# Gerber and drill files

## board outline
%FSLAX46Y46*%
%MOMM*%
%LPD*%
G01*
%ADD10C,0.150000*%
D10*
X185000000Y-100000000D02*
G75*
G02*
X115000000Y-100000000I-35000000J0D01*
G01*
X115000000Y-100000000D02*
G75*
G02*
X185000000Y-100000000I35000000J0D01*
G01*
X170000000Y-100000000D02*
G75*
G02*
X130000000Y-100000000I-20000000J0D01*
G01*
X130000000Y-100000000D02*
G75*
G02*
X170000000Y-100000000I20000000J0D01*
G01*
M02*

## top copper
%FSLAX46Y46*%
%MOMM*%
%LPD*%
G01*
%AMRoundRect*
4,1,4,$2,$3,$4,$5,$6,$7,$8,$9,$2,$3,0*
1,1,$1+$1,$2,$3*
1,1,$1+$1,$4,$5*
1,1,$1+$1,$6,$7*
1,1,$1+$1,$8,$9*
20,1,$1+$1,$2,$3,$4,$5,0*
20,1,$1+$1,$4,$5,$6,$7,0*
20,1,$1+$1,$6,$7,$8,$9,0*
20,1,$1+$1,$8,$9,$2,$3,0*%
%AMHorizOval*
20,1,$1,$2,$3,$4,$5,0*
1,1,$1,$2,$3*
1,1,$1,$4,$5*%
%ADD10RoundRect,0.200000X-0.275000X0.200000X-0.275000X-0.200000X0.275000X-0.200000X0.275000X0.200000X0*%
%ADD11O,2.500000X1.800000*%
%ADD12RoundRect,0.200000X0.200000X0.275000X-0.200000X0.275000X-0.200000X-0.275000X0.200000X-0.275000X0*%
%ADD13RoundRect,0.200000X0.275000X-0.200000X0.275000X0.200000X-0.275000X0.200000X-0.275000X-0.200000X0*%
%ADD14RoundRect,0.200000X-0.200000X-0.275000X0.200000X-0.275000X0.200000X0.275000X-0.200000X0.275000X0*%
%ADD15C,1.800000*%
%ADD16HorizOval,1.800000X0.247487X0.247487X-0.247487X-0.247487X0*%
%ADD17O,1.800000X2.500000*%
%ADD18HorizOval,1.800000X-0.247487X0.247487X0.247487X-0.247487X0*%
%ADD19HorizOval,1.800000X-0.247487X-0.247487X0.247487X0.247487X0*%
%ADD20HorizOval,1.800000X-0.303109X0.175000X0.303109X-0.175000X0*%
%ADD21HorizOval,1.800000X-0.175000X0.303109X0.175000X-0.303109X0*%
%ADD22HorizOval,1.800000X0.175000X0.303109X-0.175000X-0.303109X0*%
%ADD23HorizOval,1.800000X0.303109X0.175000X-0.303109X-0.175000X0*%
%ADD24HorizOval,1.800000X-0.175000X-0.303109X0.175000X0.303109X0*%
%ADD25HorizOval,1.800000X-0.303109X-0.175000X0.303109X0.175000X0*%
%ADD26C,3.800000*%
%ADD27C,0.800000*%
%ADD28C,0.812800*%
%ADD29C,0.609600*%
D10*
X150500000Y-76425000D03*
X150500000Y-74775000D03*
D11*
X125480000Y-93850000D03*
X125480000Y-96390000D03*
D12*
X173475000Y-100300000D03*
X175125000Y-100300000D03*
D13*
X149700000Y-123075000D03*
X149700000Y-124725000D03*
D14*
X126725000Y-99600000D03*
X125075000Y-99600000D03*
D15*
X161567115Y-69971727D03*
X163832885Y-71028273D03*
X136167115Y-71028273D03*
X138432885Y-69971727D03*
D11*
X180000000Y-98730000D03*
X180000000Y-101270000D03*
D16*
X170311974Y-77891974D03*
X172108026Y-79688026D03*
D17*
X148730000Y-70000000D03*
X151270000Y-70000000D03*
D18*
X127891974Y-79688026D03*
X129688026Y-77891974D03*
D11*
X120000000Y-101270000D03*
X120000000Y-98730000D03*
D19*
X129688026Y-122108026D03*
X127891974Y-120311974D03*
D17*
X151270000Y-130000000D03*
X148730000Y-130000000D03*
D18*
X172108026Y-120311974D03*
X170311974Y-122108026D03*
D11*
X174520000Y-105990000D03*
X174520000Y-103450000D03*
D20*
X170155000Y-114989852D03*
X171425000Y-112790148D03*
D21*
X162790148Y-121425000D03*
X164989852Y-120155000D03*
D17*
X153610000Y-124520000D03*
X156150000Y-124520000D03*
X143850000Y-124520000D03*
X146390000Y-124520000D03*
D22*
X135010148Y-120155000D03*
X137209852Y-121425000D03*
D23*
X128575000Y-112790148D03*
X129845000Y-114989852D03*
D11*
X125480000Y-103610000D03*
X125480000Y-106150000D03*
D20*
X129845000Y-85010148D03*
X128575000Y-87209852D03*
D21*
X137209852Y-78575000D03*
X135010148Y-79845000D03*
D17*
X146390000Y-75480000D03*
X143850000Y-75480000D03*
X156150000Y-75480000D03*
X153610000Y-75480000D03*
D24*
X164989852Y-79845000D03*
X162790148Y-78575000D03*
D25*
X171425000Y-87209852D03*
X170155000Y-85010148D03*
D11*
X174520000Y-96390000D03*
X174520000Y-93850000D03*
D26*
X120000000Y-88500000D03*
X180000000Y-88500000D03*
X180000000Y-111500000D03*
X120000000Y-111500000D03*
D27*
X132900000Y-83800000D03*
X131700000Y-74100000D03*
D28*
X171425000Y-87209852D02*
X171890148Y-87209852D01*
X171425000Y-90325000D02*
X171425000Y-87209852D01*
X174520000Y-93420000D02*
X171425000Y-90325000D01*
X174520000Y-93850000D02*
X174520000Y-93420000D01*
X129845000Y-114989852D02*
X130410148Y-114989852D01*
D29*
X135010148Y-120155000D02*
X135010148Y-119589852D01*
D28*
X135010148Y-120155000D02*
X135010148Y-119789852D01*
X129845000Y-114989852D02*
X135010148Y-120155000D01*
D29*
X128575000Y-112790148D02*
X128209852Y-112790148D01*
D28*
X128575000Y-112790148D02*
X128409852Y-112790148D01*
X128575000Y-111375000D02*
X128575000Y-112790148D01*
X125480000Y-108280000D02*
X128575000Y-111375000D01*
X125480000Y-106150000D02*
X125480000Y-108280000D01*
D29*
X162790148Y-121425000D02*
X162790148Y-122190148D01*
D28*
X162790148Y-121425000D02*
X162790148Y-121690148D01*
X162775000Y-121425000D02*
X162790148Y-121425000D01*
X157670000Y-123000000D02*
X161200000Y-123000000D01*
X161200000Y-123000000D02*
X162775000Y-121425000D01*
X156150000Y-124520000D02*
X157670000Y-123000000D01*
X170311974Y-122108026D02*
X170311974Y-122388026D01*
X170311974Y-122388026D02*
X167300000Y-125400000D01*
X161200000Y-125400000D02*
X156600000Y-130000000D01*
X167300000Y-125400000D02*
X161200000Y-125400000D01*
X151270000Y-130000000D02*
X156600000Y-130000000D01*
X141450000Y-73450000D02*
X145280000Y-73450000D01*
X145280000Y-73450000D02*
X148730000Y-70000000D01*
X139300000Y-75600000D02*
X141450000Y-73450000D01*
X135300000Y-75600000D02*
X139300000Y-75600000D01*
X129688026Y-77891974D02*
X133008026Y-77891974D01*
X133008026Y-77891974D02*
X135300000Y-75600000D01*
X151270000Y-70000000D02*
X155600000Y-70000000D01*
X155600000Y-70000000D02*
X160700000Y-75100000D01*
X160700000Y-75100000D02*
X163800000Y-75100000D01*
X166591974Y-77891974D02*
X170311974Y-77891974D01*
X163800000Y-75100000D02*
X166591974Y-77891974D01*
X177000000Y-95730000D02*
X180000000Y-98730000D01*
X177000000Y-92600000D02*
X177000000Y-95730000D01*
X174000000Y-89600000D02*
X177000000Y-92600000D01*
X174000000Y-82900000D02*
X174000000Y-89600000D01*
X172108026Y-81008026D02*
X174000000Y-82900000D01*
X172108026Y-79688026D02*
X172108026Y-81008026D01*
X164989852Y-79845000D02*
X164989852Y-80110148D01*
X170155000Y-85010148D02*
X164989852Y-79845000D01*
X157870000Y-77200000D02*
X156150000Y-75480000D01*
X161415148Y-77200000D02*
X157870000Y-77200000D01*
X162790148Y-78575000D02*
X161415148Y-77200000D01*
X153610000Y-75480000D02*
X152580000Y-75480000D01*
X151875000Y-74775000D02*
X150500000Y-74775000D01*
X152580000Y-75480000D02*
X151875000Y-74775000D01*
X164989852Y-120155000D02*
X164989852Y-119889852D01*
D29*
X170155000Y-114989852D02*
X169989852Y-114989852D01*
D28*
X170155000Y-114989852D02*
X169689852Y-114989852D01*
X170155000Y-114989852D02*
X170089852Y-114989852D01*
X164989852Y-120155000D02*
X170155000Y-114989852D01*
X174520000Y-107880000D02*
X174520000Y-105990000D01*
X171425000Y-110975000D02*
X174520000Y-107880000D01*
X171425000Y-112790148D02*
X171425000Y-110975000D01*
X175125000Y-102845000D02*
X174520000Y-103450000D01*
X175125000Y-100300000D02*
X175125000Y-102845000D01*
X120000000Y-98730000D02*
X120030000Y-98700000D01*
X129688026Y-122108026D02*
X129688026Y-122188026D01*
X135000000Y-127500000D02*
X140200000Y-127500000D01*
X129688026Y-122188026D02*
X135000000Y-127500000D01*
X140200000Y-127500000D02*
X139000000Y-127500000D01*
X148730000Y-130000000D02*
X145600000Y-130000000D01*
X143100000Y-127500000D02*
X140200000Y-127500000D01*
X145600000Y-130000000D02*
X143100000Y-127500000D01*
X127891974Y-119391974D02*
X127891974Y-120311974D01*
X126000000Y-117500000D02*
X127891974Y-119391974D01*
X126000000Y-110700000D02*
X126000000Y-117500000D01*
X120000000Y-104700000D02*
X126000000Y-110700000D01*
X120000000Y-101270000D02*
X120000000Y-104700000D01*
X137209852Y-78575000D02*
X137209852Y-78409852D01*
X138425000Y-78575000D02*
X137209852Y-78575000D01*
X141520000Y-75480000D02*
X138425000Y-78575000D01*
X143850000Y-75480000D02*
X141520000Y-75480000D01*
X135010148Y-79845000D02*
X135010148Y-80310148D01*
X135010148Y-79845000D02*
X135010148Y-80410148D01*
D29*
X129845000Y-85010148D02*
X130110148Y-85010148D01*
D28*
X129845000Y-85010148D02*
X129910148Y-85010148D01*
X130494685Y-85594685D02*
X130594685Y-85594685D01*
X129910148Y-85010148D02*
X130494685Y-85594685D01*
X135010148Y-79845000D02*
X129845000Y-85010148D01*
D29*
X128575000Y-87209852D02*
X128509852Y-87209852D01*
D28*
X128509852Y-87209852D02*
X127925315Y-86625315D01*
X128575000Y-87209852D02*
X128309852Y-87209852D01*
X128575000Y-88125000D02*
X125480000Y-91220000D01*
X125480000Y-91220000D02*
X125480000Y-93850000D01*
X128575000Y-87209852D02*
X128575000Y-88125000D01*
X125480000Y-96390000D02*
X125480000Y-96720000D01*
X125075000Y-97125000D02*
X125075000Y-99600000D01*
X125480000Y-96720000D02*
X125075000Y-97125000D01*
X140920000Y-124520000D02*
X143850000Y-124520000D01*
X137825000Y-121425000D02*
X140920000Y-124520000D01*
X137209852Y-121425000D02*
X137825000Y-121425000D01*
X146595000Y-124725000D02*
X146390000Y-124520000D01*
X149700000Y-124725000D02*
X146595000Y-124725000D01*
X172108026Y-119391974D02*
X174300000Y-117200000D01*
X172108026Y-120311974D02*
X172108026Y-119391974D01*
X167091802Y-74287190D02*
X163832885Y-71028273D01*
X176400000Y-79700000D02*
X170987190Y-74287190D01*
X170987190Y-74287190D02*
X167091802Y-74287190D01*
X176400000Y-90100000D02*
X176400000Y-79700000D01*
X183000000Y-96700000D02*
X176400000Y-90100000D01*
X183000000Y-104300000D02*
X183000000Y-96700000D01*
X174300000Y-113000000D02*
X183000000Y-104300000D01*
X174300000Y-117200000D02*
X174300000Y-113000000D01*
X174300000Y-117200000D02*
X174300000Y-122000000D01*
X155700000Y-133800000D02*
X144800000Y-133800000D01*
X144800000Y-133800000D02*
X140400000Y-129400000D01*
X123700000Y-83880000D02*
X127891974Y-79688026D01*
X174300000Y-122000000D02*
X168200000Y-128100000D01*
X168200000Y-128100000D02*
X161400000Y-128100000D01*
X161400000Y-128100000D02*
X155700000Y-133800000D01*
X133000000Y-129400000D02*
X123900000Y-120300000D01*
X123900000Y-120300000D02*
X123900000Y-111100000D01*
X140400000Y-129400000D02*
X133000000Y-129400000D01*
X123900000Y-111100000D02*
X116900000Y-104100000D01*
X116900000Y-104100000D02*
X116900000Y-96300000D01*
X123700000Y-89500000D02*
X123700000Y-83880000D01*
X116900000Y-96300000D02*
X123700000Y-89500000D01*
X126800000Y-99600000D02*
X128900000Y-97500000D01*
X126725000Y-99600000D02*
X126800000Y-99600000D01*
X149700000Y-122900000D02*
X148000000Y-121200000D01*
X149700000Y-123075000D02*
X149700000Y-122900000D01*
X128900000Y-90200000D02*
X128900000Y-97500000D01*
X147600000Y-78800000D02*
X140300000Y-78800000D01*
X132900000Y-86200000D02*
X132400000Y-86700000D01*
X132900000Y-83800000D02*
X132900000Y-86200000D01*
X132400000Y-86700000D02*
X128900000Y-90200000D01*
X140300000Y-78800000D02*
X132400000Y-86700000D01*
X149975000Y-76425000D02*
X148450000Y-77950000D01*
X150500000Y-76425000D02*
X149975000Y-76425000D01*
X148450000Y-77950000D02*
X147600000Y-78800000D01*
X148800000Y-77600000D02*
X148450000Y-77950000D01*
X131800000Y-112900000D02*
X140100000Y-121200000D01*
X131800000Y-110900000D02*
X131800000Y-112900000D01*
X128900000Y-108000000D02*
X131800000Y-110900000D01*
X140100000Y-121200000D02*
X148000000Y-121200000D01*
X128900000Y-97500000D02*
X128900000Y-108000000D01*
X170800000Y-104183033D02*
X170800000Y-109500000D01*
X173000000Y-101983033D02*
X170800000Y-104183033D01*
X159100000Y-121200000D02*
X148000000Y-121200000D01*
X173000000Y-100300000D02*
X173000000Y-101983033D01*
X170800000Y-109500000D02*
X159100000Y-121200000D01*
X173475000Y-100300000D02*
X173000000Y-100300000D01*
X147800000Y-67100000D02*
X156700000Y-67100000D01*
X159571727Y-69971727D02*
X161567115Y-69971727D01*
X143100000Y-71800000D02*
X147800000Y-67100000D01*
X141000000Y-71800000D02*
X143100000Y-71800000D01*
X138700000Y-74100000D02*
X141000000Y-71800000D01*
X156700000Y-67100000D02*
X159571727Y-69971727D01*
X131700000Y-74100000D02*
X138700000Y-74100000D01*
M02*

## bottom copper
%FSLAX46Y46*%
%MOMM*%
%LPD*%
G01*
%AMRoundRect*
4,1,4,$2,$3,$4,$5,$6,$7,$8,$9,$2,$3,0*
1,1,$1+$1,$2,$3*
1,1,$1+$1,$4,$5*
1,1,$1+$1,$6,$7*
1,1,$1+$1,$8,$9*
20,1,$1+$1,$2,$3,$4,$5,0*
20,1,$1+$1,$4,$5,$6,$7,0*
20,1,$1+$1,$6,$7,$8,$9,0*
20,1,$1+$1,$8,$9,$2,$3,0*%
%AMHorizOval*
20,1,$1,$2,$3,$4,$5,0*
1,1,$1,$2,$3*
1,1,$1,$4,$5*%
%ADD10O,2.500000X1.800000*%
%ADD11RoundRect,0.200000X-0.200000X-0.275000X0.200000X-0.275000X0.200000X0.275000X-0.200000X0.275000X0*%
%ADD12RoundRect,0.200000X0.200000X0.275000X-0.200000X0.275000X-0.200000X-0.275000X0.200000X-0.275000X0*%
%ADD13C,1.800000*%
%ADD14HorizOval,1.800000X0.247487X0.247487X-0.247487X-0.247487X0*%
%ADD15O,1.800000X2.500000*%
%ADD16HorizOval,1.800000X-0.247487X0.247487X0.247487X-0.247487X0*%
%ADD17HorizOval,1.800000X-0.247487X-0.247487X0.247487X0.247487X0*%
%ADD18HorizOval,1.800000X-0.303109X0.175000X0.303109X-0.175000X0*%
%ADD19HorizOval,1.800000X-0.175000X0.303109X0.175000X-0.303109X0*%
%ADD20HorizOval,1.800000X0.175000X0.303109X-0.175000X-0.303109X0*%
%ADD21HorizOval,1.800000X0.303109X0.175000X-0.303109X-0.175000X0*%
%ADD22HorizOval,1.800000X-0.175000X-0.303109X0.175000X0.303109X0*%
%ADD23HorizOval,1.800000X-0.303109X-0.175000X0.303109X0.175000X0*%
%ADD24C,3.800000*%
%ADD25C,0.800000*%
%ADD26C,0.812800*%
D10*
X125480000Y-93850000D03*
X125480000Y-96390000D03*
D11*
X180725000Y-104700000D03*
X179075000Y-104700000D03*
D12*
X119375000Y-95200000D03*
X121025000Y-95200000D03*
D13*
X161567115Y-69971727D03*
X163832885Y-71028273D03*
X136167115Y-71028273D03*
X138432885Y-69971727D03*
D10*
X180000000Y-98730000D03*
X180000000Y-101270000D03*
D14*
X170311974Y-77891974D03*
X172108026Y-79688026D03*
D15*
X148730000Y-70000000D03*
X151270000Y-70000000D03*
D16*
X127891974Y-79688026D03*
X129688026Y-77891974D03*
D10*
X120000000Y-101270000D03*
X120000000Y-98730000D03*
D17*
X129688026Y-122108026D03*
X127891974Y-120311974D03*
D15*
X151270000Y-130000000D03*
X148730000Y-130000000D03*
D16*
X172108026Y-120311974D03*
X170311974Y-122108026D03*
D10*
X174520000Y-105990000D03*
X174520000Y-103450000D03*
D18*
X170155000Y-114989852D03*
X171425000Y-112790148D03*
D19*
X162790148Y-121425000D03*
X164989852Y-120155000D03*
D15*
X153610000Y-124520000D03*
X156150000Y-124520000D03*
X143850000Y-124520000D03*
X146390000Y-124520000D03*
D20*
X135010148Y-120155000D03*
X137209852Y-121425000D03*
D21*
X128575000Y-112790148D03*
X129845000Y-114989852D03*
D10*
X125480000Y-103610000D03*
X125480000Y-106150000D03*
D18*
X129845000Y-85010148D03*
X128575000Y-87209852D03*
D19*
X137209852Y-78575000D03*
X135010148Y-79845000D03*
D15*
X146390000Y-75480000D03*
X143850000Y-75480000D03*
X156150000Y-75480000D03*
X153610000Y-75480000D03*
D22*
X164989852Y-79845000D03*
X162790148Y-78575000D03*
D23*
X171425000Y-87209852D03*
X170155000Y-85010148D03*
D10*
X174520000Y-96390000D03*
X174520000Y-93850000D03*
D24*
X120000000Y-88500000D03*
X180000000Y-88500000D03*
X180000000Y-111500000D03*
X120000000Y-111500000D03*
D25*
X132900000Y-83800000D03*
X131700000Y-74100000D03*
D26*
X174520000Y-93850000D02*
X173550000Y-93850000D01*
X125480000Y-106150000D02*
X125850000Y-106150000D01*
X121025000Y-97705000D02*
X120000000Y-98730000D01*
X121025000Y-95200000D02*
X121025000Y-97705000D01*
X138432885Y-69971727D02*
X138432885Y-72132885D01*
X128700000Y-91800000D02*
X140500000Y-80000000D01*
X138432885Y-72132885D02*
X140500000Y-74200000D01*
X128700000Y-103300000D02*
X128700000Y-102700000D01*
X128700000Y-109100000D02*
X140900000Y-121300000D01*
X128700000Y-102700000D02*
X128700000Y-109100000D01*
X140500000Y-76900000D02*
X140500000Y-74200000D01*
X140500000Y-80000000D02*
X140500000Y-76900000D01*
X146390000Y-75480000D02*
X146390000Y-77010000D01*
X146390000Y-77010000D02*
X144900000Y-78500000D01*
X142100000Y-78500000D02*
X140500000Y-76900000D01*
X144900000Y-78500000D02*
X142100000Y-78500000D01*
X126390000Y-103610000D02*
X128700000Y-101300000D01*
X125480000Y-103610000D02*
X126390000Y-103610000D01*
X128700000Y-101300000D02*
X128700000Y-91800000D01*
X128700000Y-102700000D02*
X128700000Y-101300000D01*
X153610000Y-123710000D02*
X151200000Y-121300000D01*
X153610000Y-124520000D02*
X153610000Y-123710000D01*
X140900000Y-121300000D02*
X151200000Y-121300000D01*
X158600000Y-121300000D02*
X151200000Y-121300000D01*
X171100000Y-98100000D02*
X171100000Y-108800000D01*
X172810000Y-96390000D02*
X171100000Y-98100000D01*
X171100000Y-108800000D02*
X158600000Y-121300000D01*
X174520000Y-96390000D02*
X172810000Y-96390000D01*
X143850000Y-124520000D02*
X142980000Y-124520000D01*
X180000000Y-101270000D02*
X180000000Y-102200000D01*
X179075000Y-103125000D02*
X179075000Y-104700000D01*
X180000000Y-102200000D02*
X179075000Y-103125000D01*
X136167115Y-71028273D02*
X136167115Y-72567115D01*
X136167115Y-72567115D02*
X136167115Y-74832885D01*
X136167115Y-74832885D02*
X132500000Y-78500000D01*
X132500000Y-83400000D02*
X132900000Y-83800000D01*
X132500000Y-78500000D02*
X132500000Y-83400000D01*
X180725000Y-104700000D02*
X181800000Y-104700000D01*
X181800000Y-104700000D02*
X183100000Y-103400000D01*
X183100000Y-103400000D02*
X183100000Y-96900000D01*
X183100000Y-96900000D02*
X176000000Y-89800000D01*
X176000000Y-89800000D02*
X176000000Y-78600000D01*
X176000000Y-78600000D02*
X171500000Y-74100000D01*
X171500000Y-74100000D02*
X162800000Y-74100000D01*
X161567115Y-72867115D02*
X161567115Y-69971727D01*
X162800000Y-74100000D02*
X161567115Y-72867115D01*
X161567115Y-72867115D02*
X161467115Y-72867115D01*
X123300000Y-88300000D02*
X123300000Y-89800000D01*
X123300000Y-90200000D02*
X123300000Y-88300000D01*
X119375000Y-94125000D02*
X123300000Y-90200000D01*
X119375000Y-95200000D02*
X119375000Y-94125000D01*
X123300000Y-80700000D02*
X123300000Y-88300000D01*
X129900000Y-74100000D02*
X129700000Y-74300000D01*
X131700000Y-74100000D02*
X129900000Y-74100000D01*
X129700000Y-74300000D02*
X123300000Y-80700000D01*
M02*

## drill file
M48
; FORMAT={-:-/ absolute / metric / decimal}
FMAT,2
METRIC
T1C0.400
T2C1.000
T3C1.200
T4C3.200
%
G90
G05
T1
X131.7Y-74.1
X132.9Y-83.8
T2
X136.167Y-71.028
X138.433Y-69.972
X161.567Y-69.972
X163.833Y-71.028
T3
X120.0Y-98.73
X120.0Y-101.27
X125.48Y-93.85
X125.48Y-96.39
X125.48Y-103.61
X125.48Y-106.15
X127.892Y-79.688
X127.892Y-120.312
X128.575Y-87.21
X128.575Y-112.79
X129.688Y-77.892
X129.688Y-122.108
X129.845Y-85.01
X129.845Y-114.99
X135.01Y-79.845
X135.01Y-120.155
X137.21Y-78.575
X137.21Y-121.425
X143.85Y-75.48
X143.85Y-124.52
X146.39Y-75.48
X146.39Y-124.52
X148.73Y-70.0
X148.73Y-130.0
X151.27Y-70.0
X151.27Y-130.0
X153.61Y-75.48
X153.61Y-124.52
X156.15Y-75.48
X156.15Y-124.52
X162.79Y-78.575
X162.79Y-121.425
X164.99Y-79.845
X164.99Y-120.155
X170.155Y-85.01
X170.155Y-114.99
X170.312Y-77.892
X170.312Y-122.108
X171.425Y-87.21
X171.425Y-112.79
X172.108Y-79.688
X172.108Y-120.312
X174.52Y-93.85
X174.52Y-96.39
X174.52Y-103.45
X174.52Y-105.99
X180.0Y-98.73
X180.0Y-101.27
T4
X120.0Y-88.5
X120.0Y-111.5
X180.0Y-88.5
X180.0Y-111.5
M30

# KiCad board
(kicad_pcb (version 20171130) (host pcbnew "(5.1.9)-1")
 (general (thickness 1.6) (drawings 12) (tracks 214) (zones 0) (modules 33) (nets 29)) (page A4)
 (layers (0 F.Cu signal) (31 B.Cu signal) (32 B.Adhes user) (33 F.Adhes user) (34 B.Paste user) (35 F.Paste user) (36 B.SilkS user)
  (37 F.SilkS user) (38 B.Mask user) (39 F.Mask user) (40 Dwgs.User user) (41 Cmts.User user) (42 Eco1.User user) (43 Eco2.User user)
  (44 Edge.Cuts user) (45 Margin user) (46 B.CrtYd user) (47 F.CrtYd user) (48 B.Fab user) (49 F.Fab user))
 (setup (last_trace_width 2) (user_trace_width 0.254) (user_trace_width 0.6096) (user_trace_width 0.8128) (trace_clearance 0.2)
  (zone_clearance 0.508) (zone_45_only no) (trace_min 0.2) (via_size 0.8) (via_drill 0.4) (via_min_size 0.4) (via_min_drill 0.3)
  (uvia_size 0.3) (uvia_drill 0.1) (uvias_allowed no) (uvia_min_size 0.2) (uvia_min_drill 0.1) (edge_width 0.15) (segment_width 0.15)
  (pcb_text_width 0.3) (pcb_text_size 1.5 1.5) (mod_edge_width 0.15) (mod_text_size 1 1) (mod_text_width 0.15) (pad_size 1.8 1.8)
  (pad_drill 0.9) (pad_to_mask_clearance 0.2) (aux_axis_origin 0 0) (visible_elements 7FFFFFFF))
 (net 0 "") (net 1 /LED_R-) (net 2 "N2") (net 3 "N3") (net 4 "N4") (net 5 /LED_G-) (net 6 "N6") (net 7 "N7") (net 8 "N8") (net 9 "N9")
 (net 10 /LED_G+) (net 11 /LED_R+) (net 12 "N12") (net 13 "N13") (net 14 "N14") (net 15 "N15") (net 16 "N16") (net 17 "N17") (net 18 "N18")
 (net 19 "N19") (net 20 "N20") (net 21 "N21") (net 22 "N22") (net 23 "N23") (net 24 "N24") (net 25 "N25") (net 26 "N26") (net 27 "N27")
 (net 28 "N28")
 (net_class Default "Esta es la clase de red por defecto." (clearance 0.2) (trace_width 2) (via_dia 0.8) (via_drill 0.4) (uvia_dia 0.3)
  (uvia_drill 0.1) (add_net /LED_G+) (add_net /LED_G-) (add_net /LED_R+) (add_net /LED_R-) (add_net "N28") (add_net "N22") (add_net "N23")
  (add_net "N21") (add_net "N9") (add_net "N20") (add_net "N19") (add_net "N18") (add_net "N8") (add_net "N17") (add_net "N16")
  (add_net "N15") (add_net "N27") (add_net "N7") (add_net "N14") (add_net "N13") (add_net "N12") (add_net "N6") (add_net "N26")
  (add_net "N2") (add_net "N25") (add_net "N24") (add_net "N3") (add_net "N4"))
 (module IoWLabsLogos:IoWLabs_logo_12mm (layer B.Cu) (at 162.1 128.1 18)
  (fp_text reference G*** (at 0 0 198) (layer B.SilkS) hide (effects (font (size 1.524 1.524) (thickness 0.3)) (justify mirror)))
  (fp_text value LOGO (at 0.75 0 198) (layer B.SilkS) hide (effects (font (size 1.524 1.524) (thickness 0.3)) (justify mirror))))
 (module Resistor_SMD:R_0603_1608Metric (layer F.Cu) (at 150.5 75.6 270)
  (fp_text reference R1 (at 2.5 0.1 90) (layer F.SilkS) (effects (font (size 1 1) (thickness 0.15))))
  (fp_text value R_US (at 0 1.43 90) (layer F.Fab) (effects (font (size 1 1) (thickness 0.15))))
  (pad 2 smd roundrect (at 0.825 0 270) (size 0.8 0.95) (layers F.Cu F.Paste F.Mask) (roundrect_rratio 0.25) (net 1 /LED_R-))
  (pad 1 smd roundrect (at -0.825 0 270) (size 0.8 0.95) (layers F.Cu F.Paste F.Mask) (roundrect_rratio 0.25) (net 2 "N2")))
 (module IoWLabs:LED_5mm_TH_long (layer F.Cu) (at 125.48 95.12 90)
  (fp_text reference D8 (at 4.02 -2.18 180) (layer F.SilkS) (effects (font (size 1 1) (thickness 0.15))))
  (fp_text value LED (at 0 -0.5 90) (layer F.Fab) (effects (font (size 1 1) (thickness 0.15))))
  (pad 2 thru_hole oval (at 1.27 0 90) (size 1.8 2.5) (drill 1.2) (layers *.Cu *.Mask) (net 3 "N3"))
  (pad 1 thru_hole oval (at -1.27 0 90) (size 1.8 2.5) (drill 1.2) (layers *.Cu *.Mask) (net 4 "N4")))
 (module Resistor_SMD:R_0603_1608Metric (layer B.Cu) (at 179.9 104.7)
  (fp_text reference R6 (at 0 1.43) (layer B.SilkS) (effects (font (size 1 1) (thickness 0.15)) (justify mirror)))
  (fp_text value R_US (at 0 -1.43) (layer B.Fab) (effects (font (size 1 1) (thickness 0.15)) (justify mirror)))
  (pad 2 smd roundrect (at 0.825 0) (size 0.8 0.95) (layers B.Cu B.Paste B.Mask) (roundrect_rratio 0.25) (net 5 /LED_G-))
  (pad 1 smd roundrect (at -0.825 0) (size 0.8 0.95) (layers B.Cu B.Paste B.Mask) (roundrect_rratio 0.25) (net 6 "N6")))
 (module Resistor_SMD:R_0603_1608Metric (layer B.Cu) (at 120.2 95.2 180)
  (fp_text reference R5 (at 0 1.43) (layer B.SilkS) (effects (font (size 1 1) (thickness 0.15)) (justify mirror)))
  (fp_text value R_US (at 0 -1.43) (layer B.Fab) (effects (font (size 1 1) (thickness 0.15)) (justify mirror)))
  (pad 2 smd roundrect (at 0.825 0 180) (size 0.8 0.95) (layers B.Cu B.Paste B.Mask) (roundrect_rratio 0.25) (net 5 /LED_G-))
  (pad 1 smd roundrect (at -0.825 0 180) (size 0.8 0.95) (layers B.Cu B.Paste B.Mask) (roundrect_rratio 0.25) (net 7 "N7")))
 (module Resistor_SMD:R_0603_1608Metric (layer F.Cu) (at 174.3 100.3 180)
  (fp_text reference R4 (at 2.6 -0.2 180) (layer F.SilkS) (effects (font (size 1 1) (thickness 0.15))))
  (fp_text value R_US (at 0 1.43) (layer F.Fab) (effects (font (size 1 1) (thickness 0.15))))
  (pad 2 smd roundrect (at 0.825 0 180) (size 0.8 0.95) (layers F.Cu F.Paste F.Mask) (roundrect_rratio 0.25) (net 1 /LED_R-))
  (pad 1 smd roundrect (at -0.825 0 180) (size 0.8 0.95) (layers F.Cu F.Paste F.Mask) (roundrect_rratio 0.25) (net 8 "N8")))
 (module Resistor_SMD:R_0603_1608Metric (layer F.Cu) (at 149.7 123.9 90)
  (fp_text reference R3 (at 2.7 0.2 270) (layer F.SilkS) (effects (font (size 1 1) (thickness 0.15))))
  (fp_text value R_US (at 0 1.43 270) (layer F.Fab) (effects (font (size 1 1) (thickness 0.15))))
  (pad 2 smd roundrect (at 0.825 0 90) (size 0.8 0.95) (layers F.Cu F.Paste F.Mask) (roundrect_rratio 0.25) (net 1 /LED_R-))
  (pad 1 smd roundrect (at -0.825 0 90) (size 0.8 0.95) (layers F.Cu F.Paste F.Mask) (roundrect_rratio 0.25) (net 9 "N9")))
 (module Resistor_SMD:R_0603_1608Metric (layer F.Cu) (at 125.9 99.6)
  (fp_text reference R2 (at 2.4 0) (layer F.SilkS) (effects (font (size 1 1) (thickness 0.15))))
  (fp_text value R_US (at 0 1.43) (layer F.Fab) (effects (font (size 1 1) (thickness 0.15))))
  (pad 2 smd roundrect (at 0.825 0) (size 0.8 0.95) (layers F.Cu F.Paste F.Mask) (roundrect_rratio 0.25) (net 1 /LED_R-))
  (pad 1 smd roundrect (at -0.825 0) (size 0.8 0.95) (layers F.Cu F.Paste F.Mask) (roundrect_rratio 0.25) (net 4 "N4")))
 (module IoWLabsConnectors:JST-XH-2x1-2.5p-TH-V (layer F.Cu) (at 162.7 70.5 155)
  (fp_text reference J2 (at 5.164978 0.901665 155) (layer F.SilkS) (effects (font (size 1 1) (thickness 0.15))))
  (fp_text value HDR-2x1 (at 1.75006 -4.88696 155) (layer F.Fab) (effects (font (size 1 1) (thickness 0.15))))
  (pad 2 thru_hole circle (at 1.25 0 155) (size 1.8 1.8) (drill 1) (layers *.Cu *.Mask) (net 5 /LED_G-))
  (pad 1 thru_hole circle (at -1.25 0 155) (size 1.8 1.8) (drill 1) (layers *.Cu *.Mask) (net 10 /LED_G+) (die_length 1)))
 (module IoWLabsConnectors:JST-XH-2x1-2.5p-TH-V (layer F.Cu) (at 137.3 70.5 205)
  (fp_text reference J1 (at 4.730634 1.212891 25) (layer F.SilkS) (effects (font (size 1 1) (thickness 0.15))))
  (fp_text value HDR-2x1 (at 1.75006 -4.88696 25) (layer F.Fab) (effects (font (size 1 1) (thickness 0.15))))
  (pad 2 thru_hole circle (at 1.25 0 205) (size 1.8 1.8) (drill 1) (layers *.Cu *.Mask) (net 1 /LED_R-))
  (pad 1 thru_hole circle (at -1.25 0 205) (size 1.8 1.8) (drill 1) (layers *.Cu *.Mask) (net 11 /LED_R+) (die_length 1)))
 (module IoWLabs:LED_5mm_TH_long (layer F.Cu) (at 180 100 90)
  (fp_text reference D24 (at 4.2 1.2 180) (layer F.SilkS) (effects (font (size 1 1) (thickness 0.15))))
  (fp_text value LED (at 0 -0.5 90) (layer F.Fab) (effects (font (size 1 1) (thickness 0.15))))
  (pad 2 thru_hole oval (at 1.27 0 90) (size 1.8 2.5) (drill 1.2) (layers *.Cu *.Mask) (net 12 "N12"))
  (pad 1 thru_hole oval (at -1.27 0 90) (size 1.8 2.5) (drill 1.2) (layers *.Cu *.Mask) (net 6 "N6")))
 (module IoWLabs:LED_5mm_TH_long (layer F.Cu) (at 171.21 78.79 135)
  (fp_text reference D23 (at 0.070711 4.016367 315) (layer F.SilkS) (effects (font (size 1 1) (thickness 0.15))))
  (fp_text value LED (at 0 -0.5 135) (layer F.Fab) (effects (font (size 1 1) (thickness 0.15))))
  (pad 2 thru_hole oval (at 1.27 0 135) (size 1.8 2.5) (drill 1.2) (layers *.Cu *.Mask) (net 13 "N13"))
  (pad 1 thru_hole oval (at -1.27 0 135) (size 1.8 2.5) (drill 1.2) (layers *.Cu *.Mask) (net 12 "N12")))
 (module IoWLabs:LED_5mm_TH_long (layer F.Cu) (at 150 70 180)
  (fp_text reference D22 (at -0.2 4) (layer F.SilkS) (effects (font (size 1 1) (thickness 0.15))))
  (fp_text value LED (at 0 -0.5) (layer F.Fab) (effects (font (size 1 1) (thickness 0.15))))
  (pad 2 thru_hole oval (at 1.27 0 180) (size 1.8 2.5) (drill 1.2) (layers *.Cu *.Mask) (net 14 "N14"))
  (pad 1 thru_hole oval (at -1.27 0 180) (size 1.8 2.5) (drill 1.2) (layers *.Cu *.Mask) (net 13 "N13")))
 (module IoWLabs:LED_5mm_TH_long (layer F.Cu) (at 128.79 78.79 225)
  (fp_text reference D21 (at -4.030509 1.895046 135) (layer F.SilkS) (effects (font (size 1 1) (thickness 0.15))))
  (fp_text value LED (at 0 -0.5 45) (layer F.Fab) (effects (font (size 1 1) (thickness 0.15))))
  (pad 2 thru_hole oval (at 1.27 0 225) (size 1.8 2.5) (drill 1.2) (layers *.Cu *.Mask) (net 10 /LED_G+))
  (pad 1 thru_hole oval (at -1.27 0 225) (size 1.8 2.5) (drill 1.2) (layers *.Cu *.Mask) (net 14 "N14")))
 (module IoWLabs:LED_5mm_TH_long (layer F.Cu) (at 120 100 270)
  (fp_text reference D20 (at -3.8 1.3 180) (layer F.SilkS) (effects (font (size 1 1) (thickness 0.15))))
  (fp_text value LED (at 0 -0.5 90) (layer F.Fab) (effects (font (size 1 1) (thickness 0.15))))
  (pad 2 thru_hole oval (at 1.27 0 270) (size 1.8 2.5) (drill 1.2) (layers *.Cu *.Mask) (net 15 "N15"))
  (pad 1 thru_hole oval (at -1.27 0 270) (size 1.8 2.5) (drill 1.2) (layers *.Cu *.Mask) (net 7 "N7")))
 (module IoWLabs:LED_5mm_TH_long (layer F.Cu) (at 128.79 121.21 315)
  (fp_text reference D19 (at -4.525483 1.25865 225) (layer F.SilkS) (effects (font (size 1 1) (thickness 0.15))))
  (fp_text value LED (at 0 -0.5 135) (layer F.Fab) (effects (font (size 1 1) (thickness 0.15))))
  (pad 2 thru_hole oval (at 1.27 0 315) (size 1.8 2.5) (drill 1.2) (layers *.Cu *.Mask) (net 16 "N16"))
  (pad 1 thru_hole oval (at -1.27 0 315) (size 1.8 2.5) (drill 1.2) (layers *.Cu *.Mask) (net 15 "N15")))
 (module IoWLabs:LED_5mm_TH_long (layer F.Cu) (at 150 130)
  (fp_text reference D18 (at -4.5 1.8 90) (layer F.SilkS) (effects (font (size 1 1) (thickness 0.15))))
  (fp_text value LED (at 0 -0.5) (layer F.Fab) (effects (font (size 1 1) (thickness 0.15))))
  (pad 2 thru_hole oval (at 1.27 0) (size 1.8 2.5) (drill 1.2) (layers *.Cu *.Mask) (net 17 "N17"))
  (pad 1 thru_hole oval (at -1.27 0) (size 1.8 2.5) (drill 1.2) (layers *.Cu *.Mask) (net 16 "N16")))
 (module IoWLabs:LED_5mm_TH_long (layer F.Cu) (at 171.21 121.21 45)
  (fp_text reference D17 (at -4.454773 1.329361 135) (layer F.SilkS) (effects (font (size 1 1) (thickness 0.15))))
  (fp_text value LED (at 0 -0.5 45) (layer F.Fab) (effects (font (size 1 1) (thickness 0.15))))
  (pad 2 thru_hole oval (at 1.27 0 45) (size 1.8 2.5) (drill 1.2) (layers *.Cu *.Mask) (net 10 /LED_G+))
  (pad 1 thru_hole oval (at -1.27 0 45) (size 1.8 2.5) (drill 1.2) (layers *.Cu *.Mask) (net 17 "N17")))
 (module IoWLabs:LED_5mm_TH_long (layer F.Cu) (at 174.52 104.72 270)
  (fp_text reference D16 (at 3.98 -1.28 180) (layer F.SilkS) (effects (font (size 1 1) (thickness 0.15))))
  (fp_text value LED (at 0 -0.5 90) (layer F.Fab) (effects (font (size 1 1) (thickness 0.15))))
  (pad 2 thru_hole oval (at 1.27 0 270) (size 1.8 2.5) (drill 1.2) (layers *.Cu *.Mask) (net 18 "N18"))
  (pad 1 thru_hole oval (at -1.27 0 270) (size 1.8 2.5) (drill 1.2) (layers *.Cu *.Mask) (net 8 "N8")))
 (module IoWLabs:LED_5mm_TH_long (layer F.Cu) (at 170.79 113.89 240)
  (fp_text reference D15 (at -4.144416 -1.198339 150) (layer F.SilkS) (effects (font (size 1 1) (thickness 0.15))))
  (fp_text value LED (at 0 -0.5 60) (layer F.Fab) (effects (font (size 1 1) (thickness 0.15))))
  (pad 2 thru_hole oval (at 1.27 0 240) (size 1.8 2.5) (drill 1.2) (layers *.Cu *.Mask) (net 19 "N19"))
  (pad 1 thru_hole oval (at -1.27 0 240) (size 1.8 2.5) (drill 1.2) (layers *.Cu *.Mask) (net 18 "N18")))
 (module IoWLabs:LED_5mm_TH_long (layer F.Cu) (at 163.89 120.79 210)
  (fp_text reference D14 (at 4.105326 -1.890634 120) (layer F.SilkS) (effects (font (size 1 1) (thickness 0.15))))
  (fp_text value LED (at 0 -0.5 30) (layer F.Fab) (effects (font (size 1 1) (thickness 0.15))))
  (pad 2 thru_hole oval (at 1.27 0 210) (size 1.8 2.5) (drill 1.2) (layers *.Cu *.Mask) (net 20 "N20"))
  (pad 1 thru_hole oval (at -1.27 0 210) (size 1.8 2.5) (drill 1.2) (layers *.Cu *.Mask) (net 19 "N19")))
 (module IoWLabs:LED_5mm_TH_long (layer F.Cu) (at 154.88 124.52 180)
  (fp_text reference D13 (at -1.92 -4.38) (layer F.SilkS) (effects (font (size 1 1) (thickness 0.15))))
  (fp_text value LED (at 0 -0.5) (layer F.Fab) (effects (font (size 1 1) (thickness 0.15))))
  (pad 2 thru_hole oval (at 1.27 0 180) (size 1.8 2.5) (drill 1.2) (layers *.Cu *.Mask) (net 11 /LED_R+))
  (pad 1 thru_hole oval (at -1.27 0 180) (size 1.8 2.5) (drill 1.2) (layers *.Cu *.Mask) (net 20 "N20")))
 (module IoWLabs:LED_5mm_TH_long (layer F.Cu) (at 145.12 124.52 180)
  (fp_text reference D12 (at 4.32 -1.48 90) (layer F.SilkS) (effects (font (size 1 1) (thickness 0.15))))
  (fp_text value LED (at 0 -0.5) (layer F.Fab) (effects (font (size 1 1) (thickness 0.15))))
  (pad 2 thru_hole oval (at 1.27 0 180) (size 1.8 2.5) (drill 1.2) (layers *.Cu *.Mask) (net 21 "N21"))
  (pad 1 thru_hole oval (at -1.27 0 180) (size 1.8 2.5) (drill 1.2) (layers *.Cu *.Mask) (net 9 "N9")))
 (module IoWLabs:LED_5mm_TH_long (layer F.Cu) (at 136.11 120.79 150)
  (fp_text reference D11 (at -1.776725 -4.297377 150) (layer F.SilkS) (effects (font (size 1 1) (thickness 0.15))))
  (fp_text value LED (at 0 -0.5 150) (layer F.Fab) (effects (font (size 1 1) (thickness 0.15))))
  (pad 2 thru_hole oval (at 1.27 0 150) (size 1.8 2.5) (drill 1.2) (layers *.Cu *.Mask) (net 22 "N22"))
  (pad 1 thru_hole oval (at -1.27 0 150) (size 1.8 2.5) (drill 1.2) (layers *.Cu *.Mask) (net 21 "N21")))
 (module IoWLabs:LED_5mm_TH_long (layer F.Cu) (at 129.21 113.89 120)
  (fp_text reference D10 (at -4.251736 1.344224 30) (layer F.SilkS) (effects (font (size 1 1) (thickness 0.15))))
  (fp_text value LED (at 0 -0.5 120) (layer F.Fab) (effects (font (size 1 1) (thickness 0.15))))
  (pad 2 thru_hole oval (at 1.27 0 120) (size 1.8 2.5) (drill 1.2) (layers *.Cu *.Mask) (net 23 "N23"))
  (pad 1 thru_hole oval (at -1.27 0 120) (size 1.8 2.5) (drill 1.2) (layers *.Cu *.Mask) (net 22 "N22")))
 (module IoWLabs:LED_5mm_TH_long (layer F.Cu) (at 125.48 104.88 90)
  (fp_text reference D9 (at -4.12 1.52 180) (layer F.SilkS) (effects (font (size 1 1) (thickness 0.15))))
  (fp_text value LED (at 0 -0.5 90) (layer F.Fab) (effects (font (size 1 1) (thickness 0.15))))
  (pad 2 thru_hole oval (at 1.27 0 90) (size 1.8 2.5) (drill 1.2) (layers *.Cu *.Mask) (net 11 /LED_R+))
  (pad 1 thru_hole oval (at -1.27 0 90) (size 1.8 2.5) (drill 1.2) (layers *.Cu *.Mask) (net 23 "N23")))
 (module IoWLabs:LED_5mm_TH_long (layer F.Cu) (at 129.21 86.11 60)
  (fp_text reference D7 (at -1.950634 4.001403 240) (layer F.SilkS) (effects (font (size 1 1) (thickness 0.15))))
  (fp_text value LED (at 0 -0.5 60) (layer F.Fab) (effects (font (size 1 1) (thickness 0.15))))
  (pad 2 thru_hole oval (at 1.27 0 60) (size 1.8 2.5) (drill 1.2) (layers *.Cu *.Mask) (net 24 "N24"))
  (pad 1 thru_hole oval (at -1.27 0 60) (size 1.8 2.5) (drill 1.2) (layers *.Cu *.Mask) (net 3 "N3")))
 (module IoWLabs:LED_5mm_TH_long (layer F.Cu) (at 136.11 79.21 30)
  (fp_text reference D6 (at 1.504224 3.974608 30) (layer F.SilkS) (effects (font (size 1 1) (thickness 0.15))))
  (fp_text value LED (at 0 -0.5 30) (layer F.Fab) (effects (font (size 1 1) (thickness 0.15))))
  (pad 2 thru_hole oval (at 1.27 0 30) (size 1.8 2.5) (drill 1.2) (layers *.Cu *.Mask) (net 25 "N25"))
  (pad 1 thru_hole oval (at -1.27 0 30) (size 1.8 2.5) (drill 1.2) (layers *.Cu *.Mask) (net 24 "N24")))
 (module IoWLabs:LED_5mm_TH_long (layer F.Cu) (at 145.12 75.48)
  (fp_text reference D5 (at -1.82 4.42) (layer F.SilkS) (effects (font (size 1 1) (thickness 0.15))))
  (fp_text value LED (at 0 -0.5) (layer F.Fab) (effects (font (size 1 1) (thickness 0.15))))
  (pad 2 thru_hole oval (at 1.27 0) (size 1.8 2.5) (drill 1.2) (layers *.Cu *.Mask) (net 11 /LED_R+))
  (pad 1 thru_hole oval (at -1.27 0) (size 1.8 2.5) (drill 1.2) (layers *.Cu *.Mask) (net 25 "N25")))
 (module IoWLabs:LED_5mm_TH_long (layer F.Cu) (at 154.88 75.48)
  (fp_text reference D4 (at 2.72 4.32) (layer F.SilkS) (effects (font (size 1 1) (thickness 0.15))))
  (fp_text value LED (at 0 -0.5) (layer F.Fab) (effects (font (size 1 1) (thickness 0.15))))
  (pad 2 thru_hole oval (at 1.27 0) (size 1.8 2.5) (drill 1.2) (layers *.Cu *.Mask) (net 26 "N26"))
  (pad 1 thru_hole oval (at -1.27 0) (size 1.8 2.5) (drill 1.2) (layers *.Cu *.Mask) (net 2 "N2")))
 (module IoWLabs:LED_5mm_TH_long (layer F.Cu) (at 163.89 79.21 330)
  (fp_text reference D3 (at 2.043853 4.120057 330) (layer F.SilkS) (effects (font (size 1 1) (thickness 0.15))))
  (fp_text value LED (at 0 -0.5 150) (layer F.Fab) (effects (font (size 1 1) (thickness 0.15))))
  (pad 2 thru_hole oval (at 1.27 0 330) (size 1.8 2.5) (drill 1.2) (layers *.Cu *.Mask) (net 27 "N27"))
  (pad 1 thru_hole oval (at -1.27 0 330) (size 1.8 2.5) (drill 1.2) (layers *.Cu *.Mask) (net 26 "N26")))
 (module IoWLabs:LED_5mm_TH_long (layer F.Cu) (at 170.79 86.11 300)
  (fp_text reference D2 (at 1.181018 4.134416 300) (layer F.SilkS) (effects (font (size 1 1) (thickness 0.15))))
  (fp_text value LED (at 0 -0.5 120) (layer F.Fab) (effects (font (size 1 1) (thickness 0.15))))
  (pad 2 thru_hole oval (at 1.27 0 300) (size 1.8 2.5) (drill 1.2) (layers *.Cu *.Mask) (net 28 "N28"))
  (pad 1 thru_hole oval (at -1.27 0 300) (size 1.8 2.5) (drill 1.2) (layers *.Cu *.Mask) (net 27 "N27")))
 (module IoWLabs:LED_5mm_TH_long (layer F.Cu) (at 174.52 95.12 270)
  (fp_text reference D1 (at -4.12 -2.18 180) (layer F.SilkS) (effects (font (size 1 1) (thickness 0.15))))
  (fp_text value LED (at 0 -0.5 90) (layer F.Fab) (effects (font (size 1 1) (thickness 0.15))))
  (pad 2 thru_hole oval (at 1.27 0 270) (size 1.8 2.5) (drill 1.2) (layers *.Cu *.Mask) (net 11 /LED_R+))
  (pad 1 thru_hole oval (at -1.27 0 270) (size 1.8 2.5) (drill 1.2) (layers *.Cu *.Mask) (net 28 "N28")))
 (gr_circle (center 150 100) (end 185 100) (layer Edge.Cuts) (width 0.15))
 (gr_circle (center 150 100) (end 170 100) (layer Edge.Cuts) (width 0.15))
 (via (at 120 88.5) (size 3.8) (drill 3.2) (layers F.Cu B.Cu) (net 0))
 (via (at 180 88.5) (size 3.8) (drill 3.2) (layers F.Cu B.Cu) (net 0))
 (via (at 180 111.5) (size 3.8) (drill 3.2) (layers F.Cu B.Cu) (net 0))
 (via (at 120 111.5) (size 3.8) (drill 3.2) (layers F.Cu B.Cu) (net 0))
 (segment (start 171.425 87.209852) (end 171.890148 87.209852) (width 0.8128) (layer F.Cu) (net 28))
 (segment (start 174.52 93.85) (end 173.55 93.85) (width 0.8128) (layer B.Cu) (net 28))
 (segment (start 171.425 90.325) (end 171.425 87.209852) (width 0.8128) (layer F.Cu) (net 28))
 (segment (start 174.52 93.42) (end 171.425 90.325) (width 0.8128) (layer F.Cu) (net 28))
 (segment (start 174.52 93.85) (end 174.52 93.42) (width 0.8128) (layer F.Cu) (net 28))
 (segment (start 129.845 114.989852) (end 130.410148 114.989852) (width 0.8128) (layer F.Cu) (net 22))
 (segment (start 135.010148 120.155) (end 135.010148 119.589852) (width 0.6096) (layer F.Cu) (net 22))
 (segment (start 135.010148 120.155) (end 135.010148 119.789852) (width 0.8128) (layer F.Cu) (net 22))
 (segment (start 129.845 114.989852) (end 135.010148 120.155) (width 0.8128) (layer F.Cu) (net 22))
 (segment (start 128.575 112.790148) (end 128.209852 112.790148) (width 0.6096) (layer F.Cu) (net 23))
 (segment (start 128.575 112.790148) (end 128.409852 112.790148) (width 0.8128) (layer F.Cu) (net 23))
 (segment (start 125.48 106.15) (end 125.85 106.15) (width 0.8128) (layer B.Cu) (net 23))
 (segment (start 128.575 111.375) (end 128.575 112.790148) (width 0.8128) (layer F.Cu) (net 23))
 (segment (start 125.48 108.28) (end 128.575 111.375) (width 0.8128) (layer F.Cu) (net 23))
 (segment (start 125.48 106.15) (end 125.48 108.28) (width 0.8128) (layer F.Cu) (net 23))
 (segment (start 162.790148 121.425) (end 162.790148 122.190148) (width 0.6096) (layer F.Cu) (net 20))
 (segment (start 162.790148 121.425) (end 162.790148 121.690148) (width 0.8128) (layer F.Cu) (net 20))
 (segment (start 162.775 121.425) (end 162.790148 121.425) (width 0.8128) (layer F.Cu) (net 20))
 (segment (start 157.67 123) (end 161.2 123) (width 0.8128) (layer F.Cu) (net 20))
 (segment (start 161.2 123) (end 162.775 121.425) (width 0.8128) (layer F.Cu) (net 20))
 (segment (start 156.15 124.52) (end 157.67 123) (width 0.8128) (layer F.Cu) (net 20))
 (segment (start 170.311974 122.108026) (end 170.311974 122.388026) (width 0.8128) (layer F.Cu) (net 17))
 (segment (start 170.311974 122.388026) (end 167.3 125.4) (width 0.8128) (layer F.Cu) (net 17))
 (segment (start 161.2 125.4) (end 156.6 130) (width 0.8128) (layer F.Cu) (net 17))
 (segment (start 167.3 125.4) (end 161.2 125.4) (width 0.8128) (layer F.Cu) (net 17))
 (segment (start 151.27 130) (end 156.6 130) (width 0.8128) (layer F.Cu) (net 17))
 (segment (start 141.45 73.45) (end 145.28 73.45) (width 0.8128) (layer F.Cu) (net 14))
 (segment (start 145.28 73.45) (end 148.73 70) (width 0.8128) (layer F.Cu) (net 14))
 (segment (start 139.3 75.6) (end 141.45 73.45) (width 0.8128) (layer F.Cu) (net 14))
 (segment (start 135.3 75.6) (end 139.3 75.6) (width 0.8128) (layer F.Cu) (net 14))
 (segment (start 129.688026 77.891974) (end 133.008026 77.891974) (width 0.8128) (layer F.Cu) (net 14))
 (segment (start 133.008026 77.891974) (end 135.3 75.6) (width 0.8128) (layer F.Cu) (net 14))
 (segment (start 151.27 70) (end 155.6 70) (width 0.8128) (layer F.Cu) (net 13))
 (segment (start 155.6 70) (end 160.7 75.1) (width 0.8128) (layer F.Cu) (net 13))
 (segment (start 160.7 75.1) (end 163.8 75.1) (width 0.8128) (layer F.Cu) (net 13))
 (segment (start 166.591974 77.891974) (end 170.311974 77.891974) (width 0.8128) (layer F.Cu) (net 13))
 (segment (start 163.8 75.1) (end 166.591974 77.891974) (width 0.8128) (layer F.Cu) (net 13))
 (segment (start 177 95.73) (end 180 98.73) (width 0.8128) (layer F.Cu) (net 12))
 (segment (start 177 92.6) (end 177 95.73) (width 0.8128) (layer F.Cu) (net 12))
 (segment (start 174 89.6) (end 177 92.6) (width 0.8128) (layer F.Cu) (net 12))
 (segment (start 174 82.9) (end 174 89.6) (width 0.8128) (layer F.Cu) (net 12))
 (segment (start 172.108026 81.008026) (end 174 82.9) (width 0.8128) (layer F.Cu) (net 12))
 (segment (start 172.108026 79.688026) (end 172.108026 81.008026) (width 0.8128) (layer F.Cu) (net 12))
 (segment (start 164.989852 79.845) (end 164.989852 80.110148) (width 0.8128) (layer F.Cu) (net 27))
 (segment (start 170.155 85.010148) (end 164.989852 79.845) (width 0.8128) (layer F.Cu) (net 27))
 (segment (start 157.87 77.2) (end 156.15 75.48) (width 0.8128) (layer F.Cu) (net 26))
 (segment (start 161.415148 77.2) (end 157.87 77.2) (width 0.8128) (layer F.Cu) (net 26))
 (segment (start 162.790148 78.575) (end 161.415148 77.2) (width 0.8128) (layer F.Cu) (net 26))
 (segment (start 153.61 75.48) (end 152.58 75.48) (width 0.8128) (layer F.Cu) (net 2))
 (segment (start 151.875 74.775) (end 150.5 74.775) (width 0.8128) (layer F.Cu) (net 2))
 (segment (start 152.58 75.48) (end 151.875 74.775) (width 0.8128) (layer F.Cu) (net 2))
 (segment (start 164.989852 120.155) (end 164.989852 119.889852) (width 0.8128) (layer F.Cu) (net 19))
 (segment (start 170.155 114.989852) (end 169.989852 114.989852) (width 0.6096) (layer F.Cu) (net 19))
 (segment (start 170.155 114.989852) (end 169.689852 114.989852) (width 0.8128) (layer F.Cu) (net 19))
 (segment (start 170.155 114.989852) (end 170.089852 114.989852) (width 0.8128) (layer F.Cu) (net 19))
 (segment (start 164.989852 120.155) (end 170.155 114.989852) (width 0.8128) (layer F.Cu) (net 19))
 (segment (start 174.52 107.88) (end 174.52 105.99) (width 0.8128) (layer F.Cu) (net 18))
 (segment (start 171.425 110.975) (end 174.52 107.88) (width 0.8128) (layer F.Cu) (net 18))
 (segment (start 171.425 112.790148) (end 171.425 110.975) (width 0.8128) (layer F.Cu) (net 18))
 (segment (start 175.125 102.845) (end 174.52 103.45) (width 0.8128) (layer F.Cu) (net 8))
 (segment (start 175.125 100.3) (end 175.125 102.845) (width 0.8128) (layer F.Cu) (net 8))
 (segment (start 120 98.73) (end 120.03 98.7) (width 0.8128) (layer F.Cu) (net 7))
 (segment (start 121.025 97.705) (end 120 98.73) (width 0.8128) (layer B.Cu) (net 7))
 (segment (start 121.025 95.2) (end 121.025 97.705) (width 0.8128) (layer B.Cu) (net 7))
 (segment (start 129.688026 122.108026) (end 129.688026 122.188026) (width 0.8128) (layer F.Cu) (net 16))
 (segment (start 135 127.5) (end 140.2 127.5) (width 0.8128) (layer F.Cu) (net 16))
 (segment (start 129.688026 122.188026) (end 135 127.5) (width 0.8128) (layer F.Cu) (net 16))
 (segment (start 140.2 127.5) (end 139 127.5) (width 0.8128) (layer F.Cu) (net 16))
 (segment (start 148.73 130) (end 145.6 130) (width 0.8128) (layer F.Cu) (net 16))
 (segment (start 143.1 127.5) (end 140.2 127.5) (width 0.8128) (layer F.Cu) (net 16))
 (segment (start 145.6 130) (end 143.1 127.5) (width 0.8128) (layer F.Cu) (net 16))
 (segment (start 127.891974 119.391974) (end 127.891974 120.311974) (width 0.8128) (layer F.Cu) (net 15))
 (segment (start 126 117.5) (end 127.891974 119.391974) (width 0.8128) (layer F.Cu) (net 15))
 (segment (start 126 110.7) (end 126 117.5) (width 0.8128) (layer F.Cu) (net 15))
 (segment (start 120 104.7) (end 126 110.7) (width 0.8128) (layer F.Cu) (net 15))
 (segment (start 120 101.27) (end 120 104.7) (width 0.8128) (layer F.Cu) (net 15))
 (segment (start 138.432885 69.971727) (end 138.432885 72.132885) (width 0.8128) (layer B.Cu) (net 11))
 (segment (start 128.7 91.8) (end 140.5 80) (width 0.8128) (layer B.Cu) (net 11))
 (segment (start 138.432885 72.132885) (end 140.5 74.2) (width 0.8128) (layer B.Cu) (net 11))
 (segment (start 128.7 103.3) (end 128.7 102.7) (width 0.8128) (layer B.Cu) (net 11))
 (segment (start 128.7 109.1) (end 140.9 121.3) (width 0.8128) (layer B.Cu) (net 11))
 (segment (start 128.7 102.7) (end 128.7 109.1) (width 0.8128) (layer B.Cu) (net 11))
 (segment (start 140.5 76.9) (end 140.5 74.2) (width 0.8128) (layer B.Cu) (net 11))
 (segment (start 140.5 80) (end 140.5 76.9) (width 0.8128) (layer B.Cu) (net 11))
 (segment (start 146.39 75.48) (end 146.39 77.01) (width 0.8128) (layer B.Cu) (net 11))
 (segment (start 146.39 77.01) (end 144.9 78.5) (width 0.8128) (layer B.Cu) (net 11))
 (segment (start 142.1 78.5) (end 140.5 76.9) (width 0.8128) (layer B.Cu) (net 11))
 (segment (start 144.9 78.5) (end 142.1 78.5) (width 0.8128) (layer B.Cu) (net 11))
 (segment (start 126.39 103.61) (end 128.7 101.3) (width 0.8128) (layer B.Cu) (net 11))
 (segment (start 125.48 103.61) (end 126.39 103.61) (width 0.8128) (layer B.Cu) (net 11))
 (segment (start 128.7 101.3) (end 128.7 91.8) (width 0.8128) (layer B.Cu) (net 11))
 (segment (start 128.7 102.7) (end 128.7 101.3) (width 0.8128) (layer B.Cu) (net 11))
 (segment (start 153.61 123.71) (end 151.2 121.3) (width 0.8128) (layer B.Cu) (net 11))
 (segment (start 153.61 124.52) (end 153.61 123.71) (width 0.8128) (layer B.Cu) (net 11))
 (segment (start 140.9 121.3) (end 151.2 121.3) (width 0.8128) (layer B.Cu) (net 11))
 (segment (start 158.6 121.3) (end 151.2 121.3) (width 0.8128) (layer B.Cu) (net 11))
 (segment (start 171.1 98.1) (end 171.1 108.8) (width 0.8128) (layer B.Cu) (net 11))
 (segment (start 172.81 96.39) (end 171.1 98.1) (width 0.8128) (layer B.Cu) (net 11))
 (segment (start 171.1 108.8) (end 158.6 121.3) (width 0.8128) (layer B.Cu) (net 11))
 (segment (start 174.52 96.39) (end 172.81 96.39) (width 0.8128) (layer B.Cu) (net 11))
 (segment (start 137.209852 78.575) (end 137.209852 78.409852) (width 0.8128) (layer F.Cu) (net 25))
 (segment (start 138.425 78.575) (end 137.209852 78.575) (width 0.8128) (layer F.Cu) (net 25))
 (segment (start 141.52 75.48) (end 138.425 78.575) (width 0.8128) (layer F.Cu) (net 25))
 (segment (start 143.85 75.48) (end 141.52 75.48) (width 0.8128) (layer F.Cu) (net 25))
 (segment (start 135.010148 79.845) (end 135.010148 80.310148) (width 0.8128) (layer F.Cu) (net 24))
 (segment (start 135.010148 79.845) (end 135.010148 80.410148) (width 0.8128) (layer F.Cu) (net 24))
 (segment (start 129.845 85.010148) (end 130.110148 85.010148) (width 0.6096) (layer F.Cu) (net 24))
 (segment (start 129.845 85.010148) (end 129.910148 85.010148) (width 0.8128) (layer F.Cu) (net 24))
 (segment (start 130.494685 85.594685) (end 130.594685 85.594685) (width 0.8128) (layer F.Cu) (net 24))
 (segment (start 129.910148 85.010148) (end 130.494685 85.594685) (width 0.8128) (layer F.Cu) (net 24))
 (segment (start 135.010148 79.845) (end 129.845 85.010148) (width 0.8128) (layer F.Cu) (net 24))
 (segment (start 128.575 87.209852) (end 128.509852 87.209852) (width 0.6096) (layer F.Cu) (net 3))
 (segment (start 128.509852 87.209852) (end 127.925315 86.625315) (width 0.8128) (layer F.Cu) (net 3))
 (segment (start 128.575 87.209852) (end 128.309852 87.209852) (width 0.8128) (layer F.Cu) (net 3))
 (segment (start 128.575 88.125) (end 125.48 91.22) (width 0.8128) (layer F.Cu) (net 3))
 (segment (start 125.48 91.22) (end 125.48 93.85) (width 0.8128) (layer F.Cu) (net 3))
 (segment (start 128.575 87.209852) (end 128.575 88.125) (width 0.8128) (layer F.Cu) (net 3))
 (segment (start 125.48 96.39) (end 125.48 96.72) (width 0.8128) (layer F.Cu) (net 4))
 (segment (start 125.075 97.125) (end 125.075 99.6) (width 0.8128) (layer F.Cu) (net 4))
 (segment (start 125.48 96.72) (end 125.075 97.125) (width 0.8128) (layer F.Cu) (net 4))
 (segment (start 143.85 124.52) (end 142.98 124.52) (width 0.8128) (layer B.Cu) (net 21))
 (segment (start 140.92 124.52) (end 143.85 124.52) (width 0.8128) (layer F.Cu) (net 21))
 (segment (start 137.825 121.425) (end 140.92 124.52) (width 0.8128) (layer F.Cu) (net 21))
 (segment (start 137.209852 121.425) (end 137.825 121.425) (width 0.8128) (layer F.Cu) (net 21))
 (segment (start 146.595 124.725) (end 146.39 124.52) (width 0.8128) (layer F.Cu) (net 9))
 (segment (start 149.7 124.725) (end 146.595 124.725) (width 0.8128) (layer F.Cu) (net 9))
 (segment (start 172.108026 119.391974) (end 174.3 117.2) (width 0.8128) (layer F.Cu) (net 10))
 (segment (start 172.108026 120.311974) (end 172.108026 119.391974) (width 0.8128) (layer F.Cu) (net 10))
 (segment (start 167.091802 74.28719) (end 163.832885 71.028273) (width 0.8128) (layer F.Cu) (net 10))
 (segment (start 176.4 79.7) (end 170.98719 74.28719) (width 0.8128) (layer F.Cu) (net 10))
 (segment (start 170.98719 74.28719) (end 167.091802 74.28719) (width 0.8128) (layer F.Cu) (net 10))
 (segment (start 176.4 90.1) (end 176.4 79.7) (width 0.8128) (layer F.Cu) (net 10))
 (segment (start 183 96.7) (end 176.4 90.1) (width 0.8128) (layer F.Cu) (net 10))
 (segment (start 183 104.3) (end 183 96.7) (width 0.8128) (layer F.Cu) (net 10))
 (segment (start 174.3 113) (end 183 104.3) (width 0.8128) (layer F.Cu) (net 10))
 (segment (start 174.3 117.2) (end 174.3 113) (width 0.8128) (layer F.Cu) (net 10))
 (segment (start 174.3 117.2) (end 174.3 122) (width 0.8128) (layer F.Cu) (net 10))
 (segment (start 155.7 133.8) (end 144.8 133.8) (width 0.8128) (layer F.Cu) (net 10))
 (segment (start 144.8 133.8) (end 140.4 129.4) (width 0.8128) (layer F.Cu) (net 10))
 (segment (start 123.7 83.88) (end 127.891974 79.688026) (width 0.8128) (layer F.Cu) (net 10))
 (segment (start 174.3 122) (end 168.2 128.1) (width 0.8128) (layer F.Cu) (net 10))
 (segment (start 168.2 128.1) (end 161.4 128.1) (width 0.8128) (layer F.Cu) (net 10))
 (segment (start 161.4 128.1) (end 155.7 133.8) (width 0.8128) (layer F.Cu) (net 10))
 (segment (start 133 129.4) (end 123.9 120.3) (width 0.8128) (layer F.Cu) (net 10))
 (segment (start 123.9 120.3) (end 123.9 111.1) (width 0.8128) (layer F.Cu) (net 10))
 (segment (start 140.4 129.4) (end 133 129.4) (width 0.8128) (layer F.Cu) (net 10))
 (segment (start 123.9 111.1) (end 116.9 104.1) (width 0.8128) (layer F.Cu) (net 10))
 (segment (start 116.9 104.1) (end 116.9 96.3) (width 0.8128) (layer F.Cu) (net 10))
 (segment (start 123.7 89.5) (end 123.7 83.88) (width 0.8128) (layer F.Cu) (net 10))
 (segment (start 116.9 96.3) (end 123.7 89.5) (width 0.8128) (layer F.Cu) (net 10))
 (segment (start 180 101.27) (end 180 102.2) (width 0.8128) (layer B.Cu) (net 6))
 (segment (start 179.075 103.125) (end 179.075 104.7) (width 0.8128) (layer B.Cu) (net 6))
 (segment (start 180 102.2) (end 179.075 103.125) (width 0.8128) (layer B.Cu) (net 6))
 (segment (start 126.8 99.6) (end 128.9 97.5) (width 0.8128) (layer F.Cu) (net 1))
 (segment (start 126.725 99.6) (end 126.8 99.6) (width 0.8128) (layer F.Cu) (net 1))
 (segment (start 149.7 122.9) (end 148 121.2) (width 0.8128) (layer F.Cu) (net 1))
 (segment (start 149.7 123.075) (end 149.7 122.9) (width 0.8128) (layer F.Cu) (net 1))
 (segment (start 128.9 90.2) (end 128.9 97.5) (width 0.8128) (layer F.Cu) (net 1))
 (segment (start 147.6 78.8) (end 140.3 78.8) (width 0.8128) (layer F.Cu) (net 1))
 (segment (start 136.167115 71.028273) (end 136.167115 72.567115) (width 0.8128) (layer B.Cu) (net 1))
 (segment (start 136.167115 72.567115) (end 136.167115 74.832885) (width 0.8128) (layer B.Cu) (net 1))
 (segment (start 136.167115 74.832885) (end 132.5 78.5) (width 0.8128) (layer B.Cu) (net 1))
 (via (at 132.9 83.8) (size 0.8) (drill 0.4) (layers F.Cu B.Cu) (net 1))
 (segment (start 132.5 83.4) (end 132.9 83.8) (width 0.8128) (layer B.Cu) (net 1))
 (segment (start 132.5 78.5) (end 132.5 83.4) (width 0.8128) (layer B.Cu) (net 1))
 (segment (start 132.9 86.2) (end 132.4 86.7) (width 0.8128) (layer F.Cu) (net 1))
 (segment (start 132.9 83.8) (end 132.9 86.2) (width 0.8128) (layer F.Cu) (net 1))
 (segment (start 132.4 86.7) (end 128.9 90.2) (width 0.8128) (layer F.Cu) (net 1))
 (segment (start 140.3 78.8) (end 132.4 86.7) (width 0.8128) (layer F.Cu) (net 1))
 (segment (start 149.975 76.425) (end 148.45 77.95) (width 0.8128) (layer F.Cu) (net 1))
 (segment (start 150.5 76.425) (end 149.975 76.425) (width 0.8128) (layer F.Cu) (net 1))
 (segment (start 148.45 77.95) (end 147.6 78.8) (width 0.8128) (layer F.Cu) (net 1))
 (segment (start 148.8 77.6) (end 148.45 77.95) (width 0.8128) (layer F.Cu) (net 1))
 (segment (start 131.8 112.9) (end 140.1 121.2) (width 0.8128) (layer F.Cu) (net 1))
 (segment (start 131.8 110.9) (end 131.8 112.9) (width 0.8128) (layer F.Cu) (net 1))
 (segment (start 128.9 108) (end 131.8 110.9) (width 0.8128) (layer F.Cu) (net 1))
 (segment (start 140.1 121.2) (end 148 121.2) (width 0.8128) (layer F.Cu) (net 1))
 (segment (start 128.9 97.5) (end 128.9 108) (width 0.8128) (layer F.Cu) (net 1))
 (segment (start 170.8 104.183033) (end 170.8 109.5) (width 0.8128) (layer F.Cu) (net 1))
 (segment (start 173 101.983033) (end 170.8 104.183033) (width 0.8128) (layer F.Cu) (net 1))
 (segment (start 159.1 121.2) (end 148 121.2) (width 0.8128) (layer F.Cu) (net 1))
 (segment (start 173 100.3) (end 173 101.983033) (width 0.8128) (layer F.Cu) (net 1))
 (segment (start 170.8 109.5) (end 159.1 121.2) (width 0.8128) (layer F.Cu) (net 1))
 (segment (start 173.475 100.3) (end 173 100.3) (width 0.8128) (layer F.Cu) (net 1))
 (segment (start 180.725 104.7) (end 181.8 104.7) (width 0.8128) (layer B.Cu) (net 5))
 (segment (start 181.8 104.7) (end 183.1 103.4) (width 0.8128) (layer B.Cu) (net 5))
 (segment (start 183.1 103.4) (end 183.1 96.9) (width 0.8128) (layer B.Cu) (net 5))
 (segment (start 183.1 96.9) (end 176 89.8) (width 0.8128) (layer B.Cu) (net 5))
 (segment (start 176 89.8) (end 176 78.6) (width 0.8128) (layer B.Cu) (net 5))
 (segment (start 176 78.6) (end 171.5 74.1) (width 0.8128) (layer B.Cu) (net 5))
 (segment (start 171.5 74.1) (end 162.8 74.1) (width 0.8128) (layer B.Cu) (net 5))
 (segment (start 161.567115 72.867115) (end 161.567115 69.971727) (width 0.8128) (layer B.Cu) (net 5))
 (segment (start 162.8 74.1) (end 161.567115 72.867115) (width 0.8128) (layer B.Cu) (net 5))
 (segment (start 161.567115 72.867115) (end 161.467115 72.867115) (width 0.8128) (layer B.Cu) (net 5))
 (segment (start 123.3 88.3) (end 123.3 89.8) (width 0.8128) (layer B.Cu) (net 5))
 (segment (start 123.3 90.2) (end 123.3 88.3) (width 0.8128) (layer B.Cu) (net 5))
 (segment (start 119.375 94.125) (end 123.3 90.2) (width 0.8128) (layer B.Cu) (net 5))
 (segment (start 119.375 95.2) (end 119.375 94.125) (width 0.8128) (layer B.Cu) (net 5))
 (segment (start 123.3 80.7) (end 123.3 88.3) (width 0.8128) (layer B.Cu) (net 5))
 (via (at 131.7 74.1) (size 0.8) (drill 0.4) (layers F.Cu B.Cu) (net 5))
 (segment (start 129.9 74.1) (end 129.7 74.3) (width 0.8128) (layer B.Cu) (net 5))
 (segment (start 131.7 74.1) (end 129.9 74.1) (width 0.8128) (layer B.Cu) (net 5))
 (segment (start 129.7 74.3) (end 123.3 80.7) (width 0.8128) (layer B.Cu) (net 5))
 (segment (start 147.8 67.1) (end 156.7 67.1) (width 0.8128) (layer F.Cu) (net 5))
 (segment (start 159.571727 69.971727) (end 161.567115 69.971727) (width 0.8128) (layer F.Cu) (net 5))
 (segment (start 143.1 71.8) (end 147.8 67.1) (width 0.8128) (layer F.Cu) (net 5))
 (segment (start 141 71.8) (end 143.1 71.8) (width 0.8128) (layer F.Cu) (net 5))
 (segment (start 138.7 74.1) (end 141 71.8) (width 0.8128) (layer F.Cu) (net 5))
 (segment (start 156.7 67.1) (end 159.571727 69.971727) (width 0.8128) (layer F.Cu) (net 5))
 (segment (start 131.7 74.1) (end 138.7 74.1) (width 0.8128) (layer F.Cu) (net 5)))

